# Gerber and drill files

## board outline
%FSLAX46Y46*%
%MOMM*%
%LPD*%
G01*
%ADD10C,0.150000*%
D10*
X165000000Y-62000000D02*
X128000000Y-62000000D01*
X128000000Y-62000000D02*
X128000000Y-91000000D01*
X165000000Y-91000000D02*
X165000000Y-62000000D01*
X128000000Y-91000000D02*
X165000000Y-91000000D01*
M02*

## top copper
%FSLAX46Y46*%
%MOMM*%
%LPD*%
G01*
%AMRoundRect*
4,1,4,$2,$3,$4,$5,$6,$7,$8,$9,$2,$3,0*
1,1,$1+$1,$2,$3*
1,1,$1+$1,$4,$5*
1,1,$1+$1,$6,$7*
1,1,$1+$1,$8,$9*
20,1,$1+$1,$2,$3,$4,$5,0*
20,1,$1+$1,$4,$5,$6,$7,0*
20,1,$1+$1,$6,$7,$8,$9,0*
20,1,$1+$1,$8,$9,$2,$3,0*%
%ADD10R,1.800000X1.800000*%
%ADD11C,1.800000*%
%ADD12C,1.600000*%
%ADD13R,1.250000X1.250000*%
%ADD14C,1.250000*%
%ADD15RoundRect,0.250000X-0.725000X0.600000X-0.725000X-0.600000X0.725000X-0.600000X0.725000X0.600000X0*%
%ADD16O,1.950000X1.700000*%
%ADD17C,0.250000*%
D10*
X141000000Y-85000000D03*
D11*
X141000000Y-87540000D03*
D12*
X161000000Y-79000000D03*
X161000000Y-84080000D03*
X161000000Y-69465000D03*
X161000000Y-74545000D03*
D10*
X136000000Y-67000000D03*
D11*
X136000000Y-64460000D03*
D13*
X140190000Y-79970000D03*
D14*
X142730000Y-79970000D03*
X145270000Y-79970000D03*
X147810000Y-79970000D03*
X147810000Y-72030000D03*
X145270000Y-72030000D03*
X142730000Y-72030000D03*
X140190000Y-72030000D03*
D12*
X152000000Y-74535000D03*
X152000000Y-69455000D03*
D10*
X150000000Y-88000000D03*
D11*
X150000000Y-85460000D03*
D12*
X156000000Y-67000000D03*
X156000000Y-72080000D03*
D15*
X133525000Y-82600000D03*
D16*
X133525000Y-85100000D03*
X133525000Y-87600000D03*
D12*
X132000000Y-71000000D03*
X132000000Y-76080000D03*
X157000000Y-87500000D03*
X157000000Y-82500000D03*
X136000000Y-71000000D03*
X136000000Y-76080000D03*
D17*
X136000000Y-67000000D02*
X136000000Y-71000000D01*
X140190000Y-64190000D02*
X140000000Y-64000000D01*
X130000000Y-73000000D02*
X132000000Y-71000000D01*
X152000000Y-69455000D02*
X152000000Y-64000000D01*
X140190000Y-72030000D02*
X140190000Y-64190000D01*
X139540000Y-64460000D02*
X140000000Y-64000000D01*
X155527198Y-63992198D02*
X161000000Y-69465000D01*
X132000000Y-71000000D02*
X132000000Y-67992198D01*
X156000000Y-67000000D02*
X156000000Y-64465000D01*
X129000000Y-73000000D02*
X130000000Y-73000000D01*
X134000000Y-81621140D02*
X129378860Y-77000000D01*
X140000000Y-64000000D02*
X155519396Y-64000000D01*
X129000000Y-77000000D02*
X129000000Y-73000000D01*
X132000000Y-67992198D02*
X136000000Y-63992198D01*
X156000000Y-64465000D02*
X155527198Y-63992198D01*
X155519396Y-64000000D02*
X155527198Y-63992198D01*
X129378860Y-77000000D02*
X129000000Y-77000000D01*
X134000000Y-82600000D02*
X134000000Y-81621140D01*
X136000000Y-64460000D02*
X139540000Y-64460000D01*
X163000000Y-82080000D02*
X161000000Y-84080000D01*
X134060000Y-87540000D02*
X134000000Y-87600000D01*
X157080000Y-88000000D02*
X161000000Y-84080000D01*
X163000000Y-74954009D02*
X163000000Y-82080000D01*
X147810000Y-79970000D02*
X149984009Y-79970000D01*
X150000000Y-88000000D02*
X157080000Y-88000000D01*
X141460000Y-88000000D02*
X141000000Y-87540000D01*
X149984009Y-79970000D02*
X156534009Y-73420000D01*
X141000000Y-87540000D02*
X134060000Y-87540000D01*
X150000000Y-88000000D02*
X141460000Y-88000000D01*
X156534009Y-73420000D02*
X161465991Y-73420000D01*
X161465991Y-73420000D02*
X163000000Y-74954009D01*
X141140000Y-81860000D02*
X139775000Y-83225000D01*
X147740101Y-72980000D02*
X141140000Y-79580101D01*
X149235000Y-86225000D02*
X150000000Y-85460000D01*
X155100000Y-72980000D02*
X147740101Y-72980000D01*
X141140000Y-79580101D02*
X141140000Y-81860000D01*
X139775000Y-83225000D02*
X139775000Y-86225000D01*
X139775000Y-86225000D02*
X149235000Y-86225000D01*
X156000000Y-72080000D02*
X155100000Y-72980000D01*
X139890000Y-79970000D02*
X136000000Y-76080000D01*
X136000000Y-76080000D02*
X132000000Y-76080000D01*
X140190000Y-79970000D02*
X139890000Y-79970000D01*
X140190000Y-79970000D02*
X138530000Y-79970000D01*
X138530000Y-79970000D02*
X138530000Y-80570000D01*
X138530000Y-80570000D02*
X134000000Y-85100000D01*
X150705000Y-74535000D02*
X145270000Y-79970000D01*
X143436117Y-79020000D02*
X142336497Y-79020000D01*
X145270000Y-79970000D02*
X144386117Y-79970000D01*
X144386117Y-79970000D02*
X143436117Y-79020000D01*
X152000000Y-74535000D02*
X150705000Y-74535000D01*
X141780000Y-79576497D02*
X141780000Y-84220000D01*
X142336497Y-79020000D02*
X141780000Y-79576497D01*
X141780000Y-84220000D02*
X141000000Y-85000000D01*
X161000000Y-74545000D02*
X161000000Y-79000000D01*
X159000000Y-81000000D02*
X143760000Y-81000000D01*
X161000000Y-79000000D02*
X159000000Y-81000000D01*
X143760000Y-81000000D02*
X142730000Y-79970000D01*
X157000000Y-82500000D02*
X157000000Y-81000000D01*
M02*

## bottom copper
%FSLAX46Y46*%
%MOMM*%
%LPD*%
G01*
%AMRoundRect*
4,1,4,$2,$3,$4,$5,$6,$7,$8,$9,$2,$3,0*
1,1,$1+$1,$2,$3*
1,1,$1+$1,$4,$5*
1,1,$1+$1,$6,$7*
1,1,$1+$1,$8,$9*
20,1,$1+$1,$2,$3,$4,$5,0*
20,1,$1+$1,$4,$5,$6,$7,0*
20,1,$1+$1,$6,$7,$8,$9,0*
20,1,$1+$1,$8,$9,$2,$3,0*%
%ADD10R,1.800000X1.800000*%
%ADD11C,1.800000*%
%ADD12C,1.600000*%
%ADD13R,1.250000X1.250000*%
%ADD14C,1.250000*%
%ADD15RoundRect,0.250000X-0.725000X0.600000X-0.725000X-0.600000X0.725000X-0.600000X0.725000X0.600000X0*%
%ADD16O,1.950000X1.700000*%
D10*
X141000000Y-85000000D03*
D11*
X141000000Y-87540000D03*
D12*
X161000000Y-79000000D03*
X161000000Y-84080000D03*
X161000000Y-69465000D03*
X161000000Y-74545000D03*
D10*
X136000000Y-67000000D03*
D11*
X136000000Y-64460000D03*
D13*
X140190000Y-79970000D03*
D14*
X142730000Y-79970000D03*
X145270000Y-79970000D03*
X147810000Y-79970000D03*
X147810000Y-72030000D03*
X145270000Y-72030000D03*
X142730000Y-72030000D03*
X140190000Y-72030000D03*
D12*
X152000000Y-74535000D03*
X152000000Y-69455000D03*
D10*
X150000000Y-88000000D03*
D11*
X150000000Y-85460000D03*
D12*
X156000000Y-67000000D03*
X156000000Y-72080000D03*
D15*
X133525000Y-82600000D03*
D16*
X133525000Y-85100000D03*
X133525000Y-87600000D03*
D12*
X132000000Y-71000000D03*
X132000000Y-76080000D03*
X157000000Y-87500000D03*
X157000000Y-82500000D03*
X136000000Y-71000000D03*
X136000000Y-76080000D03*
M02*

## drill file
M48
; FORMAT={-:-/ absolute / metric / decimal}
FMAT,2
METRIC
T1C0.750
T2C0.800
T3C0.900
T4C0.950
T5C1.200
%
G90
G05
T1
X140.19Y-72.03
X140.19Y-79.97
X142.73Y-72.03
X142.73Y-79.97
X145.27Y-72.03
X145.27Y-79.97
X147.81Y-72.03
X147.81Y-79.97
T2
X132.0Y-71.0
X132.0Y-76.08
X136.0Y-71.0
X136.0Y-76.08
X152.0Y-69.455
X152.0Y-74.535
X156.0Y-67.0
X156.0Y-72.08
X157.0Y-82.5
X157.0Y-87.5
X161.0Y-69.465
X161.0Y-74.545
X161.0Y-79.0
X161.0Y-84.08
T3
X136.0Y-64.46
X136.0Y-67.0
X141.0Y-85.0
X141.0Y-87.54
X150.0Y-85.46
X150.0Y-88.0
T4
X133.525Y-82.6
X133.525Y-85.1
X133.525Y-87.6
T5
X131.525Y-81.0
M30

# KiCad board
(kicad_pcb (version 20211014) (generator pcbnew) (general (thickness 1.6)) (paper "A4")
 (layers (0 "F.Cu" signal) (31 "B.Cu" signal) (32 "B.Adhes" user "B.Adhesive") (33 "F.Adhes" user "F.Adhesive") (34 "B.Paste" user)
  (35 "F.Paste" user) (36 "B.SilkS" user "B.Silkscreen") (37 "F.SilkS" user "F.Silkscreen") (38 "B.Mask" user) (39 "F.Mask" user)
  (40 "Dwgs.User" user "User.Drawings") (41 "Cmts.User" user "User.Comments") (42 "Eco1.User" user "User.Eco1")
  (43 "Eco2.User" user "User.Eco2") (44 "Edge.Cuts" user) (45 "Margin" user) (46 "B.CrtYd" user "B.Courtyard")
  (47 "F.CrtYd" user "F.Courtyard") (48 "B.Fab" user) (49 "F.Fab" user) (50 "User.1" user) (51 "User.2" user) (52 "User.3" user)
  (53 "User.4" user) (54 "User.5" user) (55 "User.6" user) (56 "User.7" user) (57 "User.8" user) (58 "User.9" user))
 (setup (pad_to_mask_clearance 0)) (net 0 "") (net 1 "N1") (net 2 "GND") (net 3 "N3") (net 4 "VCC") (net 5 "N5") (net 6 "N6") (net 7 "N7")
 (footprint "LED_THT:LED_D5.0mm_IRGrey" (layer "F.Cu") (at 141 85 -90)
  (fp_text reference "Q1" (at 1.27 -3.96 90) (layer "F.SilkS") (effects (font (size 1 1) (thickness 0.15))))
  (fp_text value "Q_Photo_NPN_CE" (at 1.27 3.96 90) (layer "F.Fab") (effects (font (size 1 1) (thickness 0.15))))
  (pad "1" thru_hole rect (at 0 0 270) (size 1.8 1.8) (drill 0.9) (layers *.Cu *.Mask) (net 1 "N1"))
  (pad "2" thru_hole circle (at 2.54 0 270) (size 1.8 1.8) (drill 0.9) (layers *.Cu *.Mask) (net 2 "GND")))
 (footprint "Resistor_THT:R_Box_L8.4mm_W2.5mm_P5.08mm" (layer "F.Cu") (at 161 79 -90)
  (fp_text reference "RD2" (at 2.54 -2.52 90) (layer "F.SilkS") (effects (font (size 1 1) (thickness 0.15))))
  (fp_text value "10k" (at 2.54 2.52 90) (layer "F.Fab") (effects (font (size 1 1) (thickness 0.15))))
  (pad "1" thru_hole circle (at 0 0 270) (size 1.6 1.6) (drill 0.8) (layers *.Cu *.Mask) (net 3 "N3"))
  (pad "2" thru_hole circle (at 5.08 0 270) (size 1.6 1.6) (drill 0.8) (layers *.Cu *.Mask) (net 2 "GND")))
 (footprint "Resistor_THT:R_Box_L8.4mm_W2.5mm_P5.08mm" (layer "F.Cu") (at 161 69.465 -90)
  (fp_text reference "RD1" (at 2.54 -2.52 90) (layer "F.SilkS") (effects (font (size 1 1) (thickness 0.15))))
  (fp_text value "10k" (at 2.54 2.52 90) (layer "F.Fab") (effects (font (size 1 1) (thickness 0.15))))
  (pad "1" thru_hole circle (at 0 0 270) (size 1.6 1.6) (drill 0.8) (layers *.Cu *.Mask) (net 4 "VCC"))
  (pad "2" thru_hole circle (at 5.08 0 270) (size 1.6 1.6) (drill 0.8) (layers *.Cu *.Mask) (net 3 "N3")))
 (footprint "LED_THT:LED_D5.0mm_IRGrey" (layer "F.Cu") (at 136 67 90)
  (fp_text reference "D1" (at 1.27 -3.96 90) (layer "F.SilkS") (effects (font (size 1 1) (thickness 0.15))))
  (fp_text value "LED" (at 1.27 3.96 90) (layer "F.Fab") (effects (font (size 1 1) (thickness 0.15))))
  (pad "1" thru_hole rect (at 0 0 90) (size 1.8 1.8) (drill 0.9) (layers *.Cu *.Mask) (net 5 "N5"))
  (pad "2" thru_hole circle (at 2.54 0 90) (size 1.8 1.8) (drill 0.9) (layers *.Cu *.Mask) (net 4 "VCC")))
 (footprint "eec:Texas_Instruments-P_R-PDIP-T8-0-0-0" (layer "F.Cu") (at 144 76 90)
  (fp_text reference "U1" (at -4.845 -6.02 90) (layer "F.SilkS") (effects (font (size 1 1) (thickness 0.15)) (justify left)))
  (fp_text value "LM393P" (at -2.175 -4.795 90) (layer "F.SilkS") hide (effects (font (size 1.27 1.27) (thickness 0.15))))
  (pad "1" thru_hole rect locked (at -3.97 -3.81 90) (size 1.25 1.25) (drill 0.75) (layers *.Cu *.Mask) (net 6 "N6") (thermal_width 0.4))
  (pad "2" thru_hole circle locked (at -3.97 -1.27 90) (size 1.25 1.25) (drill 0.75) (layers *.Cu *.Mask) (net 3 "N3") (thermal_width 0.4))
  (pad "3" thru_hole circle locked (at -3.97 1.27 90) (size 1.25 1.25) (drill 0.75) (layers *.Cu *.Mask) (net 1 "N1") (thermal_width 0.4))
  (pad "4" thru_hole circle locked (at -3.97 3.81 90) (size 1.25 1.25) (drill 0.75) (layers *.Cu *.Mask) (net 2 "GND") (thermal_width 0.4))
  (pad "5" thru_hole circle locked (at 3.97 3.81 90) (size 1.25 1.25) (drill 0.75) (layers *.Cu "B.Mask") (thermal_width 0.4))
  (pad "6" thru_hole circle locked (at 3.97 1.27 90) (size 1.25 1.25) (drill 0.75) (layers *.Cu "B.Mask") (thermal_width 0.4))
  (pad "7" thru_hole circle locked (at 3.97 -1.27 90) (size 1.25 1.25) (drill 0.75) (layers *.Cu "B.Mask") (thermal_width 0.4))
  (pad "8" thru_hole circle locked (at 3.97 -3.81 90) (size 1.25 1.25) (drill 0.75) (layers *.Cu *.Mask) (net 4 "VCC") (thermal_width 0.4)))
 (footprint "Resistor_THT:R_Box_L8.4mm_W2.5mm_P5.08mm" (layer "F.Cu") (at 152 74.535 90)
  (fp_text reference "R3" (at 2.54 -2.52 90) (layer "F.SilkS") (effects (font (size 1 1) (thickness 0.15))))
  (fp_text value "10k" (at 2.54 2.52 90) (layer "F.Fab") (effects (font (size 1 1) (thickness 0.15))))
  (pad "1" thru_hole circle (at 0 0 90) (size 1.6 1.6) (drill 0.8) (layers *.Cu *.Mask) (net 1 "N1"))
  (pad "2" thru_hole circle (at 5.08 0 90) (size 1.6 1.6) (drill 0.8) (layers *.Cu *.Mask) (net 4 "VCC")))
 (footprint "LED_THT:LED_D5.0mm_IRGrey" (layer "F.Cu") (at 150 88 90)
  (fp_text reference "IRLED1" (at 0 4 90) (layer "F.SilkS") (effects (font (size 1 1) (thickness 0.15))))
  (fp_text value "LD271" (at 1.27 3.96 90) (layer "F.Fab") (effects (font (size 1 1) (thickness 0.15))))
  (pad "1" thru_hole rect (at 0 0 90) (size 1.8 1.8) (drill 0.9) (layers *.Cu *.Mask) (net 2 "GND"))
  (pad "2" thru_hole circle (at 2.54 0 90) (size 1.8 1.8) (drill 0.9) (layers *.Cu *.Mask) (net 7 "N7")))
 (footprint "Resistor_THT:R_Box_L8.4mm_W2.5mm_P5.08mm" (layer "F.Cu") (at 156 67 -90)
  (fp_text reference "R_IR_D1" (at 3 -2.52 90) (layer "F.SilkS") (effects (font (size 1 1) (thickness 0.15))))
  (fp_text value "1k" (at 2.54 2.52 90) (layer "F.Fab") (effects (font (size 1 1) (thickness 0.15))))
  (pad "1" thru_hole circle (at 0 0 270) (size 1.6 1.6) (drill 0.8) (layers *.Cu *.Mask) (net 4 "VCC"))
  (pad "2" thru_hole circle (at 5.08 0 270) (size 1.6 1.6) (drill 0.8) (layers *.Cu *.Mask) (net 7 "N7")))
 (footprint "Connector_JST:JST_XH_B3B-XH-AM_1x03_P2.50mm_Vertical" (layer "F.Cu") (at 133.525 82.6 -90)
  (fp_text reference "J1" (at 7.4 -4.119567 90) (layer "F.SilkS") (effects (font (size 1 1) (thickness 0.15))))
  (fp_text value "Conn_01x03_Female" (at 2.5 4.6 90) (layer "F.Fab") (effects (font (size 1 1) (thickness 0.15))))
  (pad "" np_thru_hole circle (at -1.6 2 270) (size 1.2 1.2) (drill 1.2) (layers *.Cu *.Mask))
  (pad "1" thru_hole roundrect (at 0 0 270) (size 1.7 1.95) (drill 0.95) (layers *.Cu *.Mask) (roundrect_rratio 0.1470588235) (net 4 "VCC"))
  (pad "2" thru_hole oval (at 2.5 0 270) (size 1.7 1.95) (drill 0.95) (layers *.Cu *.Mask) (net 6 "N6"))
  (pad "3" thru_hole oval (at 5 0 270) (size 1.7 1.95) (drill 0.95) (layers *.Cu *.Mask) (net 2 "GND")))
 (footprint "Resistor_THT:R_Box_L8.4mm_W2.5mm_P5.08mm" (layer "F.Cu") (at 132 71 -90)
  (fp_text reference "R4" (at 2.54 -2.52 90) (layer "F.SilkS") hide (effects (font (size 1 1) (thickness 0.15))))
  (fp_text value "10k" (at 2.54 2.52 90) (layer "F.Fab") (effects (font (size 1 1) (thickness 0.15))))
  (pad "1" thru_hole circle (at 0 0 270) (size 1.6 1.6) (drill 0.8) (layers *.Cu *.Mask) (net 4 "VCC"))
  (pad "2" thru_hole circle (at 5.08 0 270) (size 1.6 1.6) (drill 0.8) (layers *.Cu *.Mask) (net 6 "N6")))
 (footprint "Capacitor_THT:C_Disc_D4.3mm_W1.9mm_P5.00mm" (layer "F.Cu") (at 157 87.5 90)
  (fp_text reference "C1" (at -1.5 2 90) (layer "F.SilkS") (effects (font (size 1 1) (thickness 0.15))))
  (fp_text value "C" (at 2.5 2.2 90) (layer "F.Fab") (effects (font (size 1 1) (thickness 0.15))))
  (pad "1" thru_hole circle (at 0 0 90) (size 1.6 1.6) (drill 0.8) (layers *.Cu *.Mask) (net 2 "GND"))
  (pad "2" thru_hole circle (at 5 0 90) (size 1.6 1.6) (drill 0.8) (layers *.Cu *.Mask) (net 3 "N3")))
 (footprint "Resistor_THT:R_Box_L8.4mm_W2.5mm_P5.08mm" (layer "F.Cu") (at 136 71 -90)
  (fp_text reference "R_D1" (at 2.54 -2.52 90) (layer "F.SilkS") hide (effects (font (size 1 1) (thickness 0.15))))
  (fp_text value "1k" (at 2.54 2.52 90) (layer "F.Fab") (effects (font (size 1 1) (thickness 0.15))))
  (pad "1" thru_hole circle (at 0 0 270) (size 1.6 1.6) (drill 0.8) (layers *.Cu *.Mask) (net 5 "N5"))
  (pad "2" thru_hole circle (at 5.08 0 270) (size 1.6 1.6) (drill 0.8) (layers *.Cu *.Mask) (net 6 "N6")))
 (gr_line (start 165 62) (end 128 62) (layer "Edge.Cuts") (width 0.15))
 (gr_line (start 128 62) (end 128 91) (layer "Edge.Cuts") (width 0.15))
 (gr_line (start 165 91) (end 165 62) (layer "Edge.Cuts") (width 0.15))
 (gr_line (start 128 91) (end 165 91) (layer "Edge.Cuts") (width 0.15))
 (segment (start 136 67) (end 136 71) (width 0.25) (layer "F.Cu") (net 5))
 (segment (start 140.19 64.19) (end 140 64) (width 0.25) (layer "F.Cu") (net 4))
 (segment (start 130 73) (end 132 71) (width 0.25) (layer "F.Cu") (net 4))
 (segment (start 152 69.455) (end 152 64) (width 0.25) (layer "F.Cu") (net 4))
 (segment (start 140.19 72.03) (end 140.19 64.19) (width 0.25) (layer "F.Cu") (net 4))
 (segment (start 139.54 64.46) (end 140 64) (width 0.25) (layer "F.Cu") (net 4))
 (segment (start 155.527198 63.992198) (end 161 69.465) (width 0.25) (layer "F.Cu") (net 4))
 (segment (start 132 71) (end 132 67.992198) (width 0.25) (layer "F.Cu") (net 4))
 (segment (start 156 67) (end 156 64.465) (width 0.25) (layer "F.Cu") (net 4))
 (segment (start 129 73) (end 130 73) (width 0.25) (layer "F.Cu") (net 4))
 (segment (start 134 81.62114) (end 129.37886 77) (width 0.25) (layer "F.Cu") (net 4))
 (segment (start 140 64) (end 155.519396 64) (width 0.25) (layer "F.Cu") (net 4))
 (segment (start 129 77) (end 129 73) (width 0.25) (layer "F.Cu") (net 4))
 (segment (start 132 67.992198) (end 136 63.992198) (width 0.25) (layer "F.Cu") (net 4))
 (segment (start 156 64.465) (end 155.527198 63.992198) (width 0.25) (layer "F.Cu") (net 4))
 (segment (start 155.519396 64) (end 155.527198 63.992198) (width 0.25) (layer "F.Cu") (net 4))
 (segment (start 129.37886 77) (end 129 77) (width 0.25) (layer "F.Cu") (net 4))
 (segment (start 134 82.6) (end 134 81.62114) (width 0.25) (layer "F.Cu") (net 4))
 (segment (start 136 64.46) (end 139.54 64.46) (width 0.25) (layer "F.Cu") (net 4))
 (segment (start 163 82.08) (end 161 84.08) (width 0.25) (layer "F.Cu") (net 2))
 (segment (start 134.06 87.54) (end 134 87.6) (width 0.25) (layer "F.Cu") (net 2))
 (segment (start 157.08 88) (end 161 84.08) (width 0.25) (layer "F.Cu") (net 2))
 (segment (start 163 74.954009) (end 163 82.08) (width 0.25) (layer "F.Cu") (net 2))
 (segment (start 147.81 79.97) (end 149.984009 79.97) (width 0.25) (layer "F.Cu") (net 2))
 (segment (start 150 88) (end 157.08 88) (width 0.25) (layer "F.Cu") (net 2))
 (segment (start 141.46 88) (end 141 87.54) (width 0.25) (layer "F.Cu") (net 2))
 (segment (start 149.984009 79.97) (end 156.534009 73.42) (width 0.25) (layer "F.Cu") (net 2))
 (segment (start 141 87.54) (end 134.06 87.54) (width 0.25) (layer "F.Cu") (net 2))
 (segment (start 150 88) (end 141.46 88) (width 0.25) (layer "F.Cu") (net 2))
 (segment (start 156.534009 73.42) (end 161.465991 73.42) (width 0.25) (layer "F.Cu") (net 2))
 (segment (start 161.465991 73.42) (end 163 74.954009) (width 0.25) (layer "F.Cu") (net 2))
 (segment (start 141.14 81.86) (end 139.775 83.225) (width 0.25) (layer "F.Cu") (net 7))
 (segment (start 147.740101 72.98) (end 141.14 79.580101) (width 0.25) (layer "F.Cu") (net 7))
 (segment (start 149.235 86.225) (end 150 85.46) (width 0.25) (layer "F.Cu") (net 7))
 (segment (start 155.1 72.98) (end 147.740101 72.98) (width 0.25) (layer "F.Cu") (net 7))
 (segment (start 141.14 79.580101) (end 141.14 81.86) (width 0.25) (layer "F.Cu") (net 7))
 (segment (start 139.775 83.225) (end 139.775 86.225) (width 0.25) (layer "F.Cu") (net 7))
 (segment (start 139.775 86.225) (end 149.235 86.225) (width 0.25) (layer "F.Cu") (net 7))
 (segment (start 156 72.08) (end 155.1 72.98) (width 0.25) (layer "F.Cu") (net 7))
 (segment (start 139.89 79.97) (end 136 76.08) (width 0.25) (layer "F.Cu") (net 6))
 (segment (start 136 76.08) (end 132 76.08) (width 0.25) (layer "F.Cu") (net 6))
 (segment (start 140.19 79.97) (end 139.89 79.97) (width 0.25) (layer "F.Cu") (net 6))
 (segment (start 140.19 79.97) (end 138.53 79.97) (width 0.25) (layer "F.Cu") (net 6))
 (segment (start 138.53 79.97) (end 138.53 80.57) (width 0.25) (layer "F.Cu") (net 6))
 (segment (start 138.53 80.57) (end 134 85.1) (width 0.25) (layer "F.Cu") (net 6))
 (segment (start 150.705 74.535) (end 145.27 79.97) (width 0.25) (layer "F.Cu") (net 1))
 (segment (start 143.436117 79.02) (end 142.336497 79.02) (width 0.25) (layer "F.Cu") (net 1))
 (segment (start 145.27 79.97) (end 144.386117 79.97) (width 0.25) (layer "F.Cu") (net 1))
 (segment (start 144.386117 79.97) (end 143.436117 79.02) (width 0.25) (layer "F.Cu") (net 1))
 (segment (start 152 74.535) (end 150.705 74.535) (width 0.25) (layer "F.Cu") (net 1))
 (segment (start 141.78 79.576497) (end 141.78 84.22) (width 0.25) (layer "F.Cu") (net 1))
 (segment (start 142.336497 79.02) (end 141.78 79.576497) (width 0.25) (layer "F.Cu") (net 1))
 (segment (start 141.78 84.22) (end 141 85) (width 0.25) (layer "F.Cu") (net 1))
 (segment (start 161 74.545) (end 161 79) (width 0.25) (layer "F.Cu") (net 3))
 (segment (start 159 81) (end 143.76 81) (width 0.25) (layer "F.Cu") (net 3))
 (segment (start 161 79) (end 159 81) (width 0.25) (layer "F.Cu") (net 3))
 (segment (start 143.76 81) (end 142.73 79.97) (width 0.25) (layer "F.Cu") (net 3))
 (segment (start 157 82.5) (end 157 81) (width 0.25) (layer "F.Cu") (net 3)))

